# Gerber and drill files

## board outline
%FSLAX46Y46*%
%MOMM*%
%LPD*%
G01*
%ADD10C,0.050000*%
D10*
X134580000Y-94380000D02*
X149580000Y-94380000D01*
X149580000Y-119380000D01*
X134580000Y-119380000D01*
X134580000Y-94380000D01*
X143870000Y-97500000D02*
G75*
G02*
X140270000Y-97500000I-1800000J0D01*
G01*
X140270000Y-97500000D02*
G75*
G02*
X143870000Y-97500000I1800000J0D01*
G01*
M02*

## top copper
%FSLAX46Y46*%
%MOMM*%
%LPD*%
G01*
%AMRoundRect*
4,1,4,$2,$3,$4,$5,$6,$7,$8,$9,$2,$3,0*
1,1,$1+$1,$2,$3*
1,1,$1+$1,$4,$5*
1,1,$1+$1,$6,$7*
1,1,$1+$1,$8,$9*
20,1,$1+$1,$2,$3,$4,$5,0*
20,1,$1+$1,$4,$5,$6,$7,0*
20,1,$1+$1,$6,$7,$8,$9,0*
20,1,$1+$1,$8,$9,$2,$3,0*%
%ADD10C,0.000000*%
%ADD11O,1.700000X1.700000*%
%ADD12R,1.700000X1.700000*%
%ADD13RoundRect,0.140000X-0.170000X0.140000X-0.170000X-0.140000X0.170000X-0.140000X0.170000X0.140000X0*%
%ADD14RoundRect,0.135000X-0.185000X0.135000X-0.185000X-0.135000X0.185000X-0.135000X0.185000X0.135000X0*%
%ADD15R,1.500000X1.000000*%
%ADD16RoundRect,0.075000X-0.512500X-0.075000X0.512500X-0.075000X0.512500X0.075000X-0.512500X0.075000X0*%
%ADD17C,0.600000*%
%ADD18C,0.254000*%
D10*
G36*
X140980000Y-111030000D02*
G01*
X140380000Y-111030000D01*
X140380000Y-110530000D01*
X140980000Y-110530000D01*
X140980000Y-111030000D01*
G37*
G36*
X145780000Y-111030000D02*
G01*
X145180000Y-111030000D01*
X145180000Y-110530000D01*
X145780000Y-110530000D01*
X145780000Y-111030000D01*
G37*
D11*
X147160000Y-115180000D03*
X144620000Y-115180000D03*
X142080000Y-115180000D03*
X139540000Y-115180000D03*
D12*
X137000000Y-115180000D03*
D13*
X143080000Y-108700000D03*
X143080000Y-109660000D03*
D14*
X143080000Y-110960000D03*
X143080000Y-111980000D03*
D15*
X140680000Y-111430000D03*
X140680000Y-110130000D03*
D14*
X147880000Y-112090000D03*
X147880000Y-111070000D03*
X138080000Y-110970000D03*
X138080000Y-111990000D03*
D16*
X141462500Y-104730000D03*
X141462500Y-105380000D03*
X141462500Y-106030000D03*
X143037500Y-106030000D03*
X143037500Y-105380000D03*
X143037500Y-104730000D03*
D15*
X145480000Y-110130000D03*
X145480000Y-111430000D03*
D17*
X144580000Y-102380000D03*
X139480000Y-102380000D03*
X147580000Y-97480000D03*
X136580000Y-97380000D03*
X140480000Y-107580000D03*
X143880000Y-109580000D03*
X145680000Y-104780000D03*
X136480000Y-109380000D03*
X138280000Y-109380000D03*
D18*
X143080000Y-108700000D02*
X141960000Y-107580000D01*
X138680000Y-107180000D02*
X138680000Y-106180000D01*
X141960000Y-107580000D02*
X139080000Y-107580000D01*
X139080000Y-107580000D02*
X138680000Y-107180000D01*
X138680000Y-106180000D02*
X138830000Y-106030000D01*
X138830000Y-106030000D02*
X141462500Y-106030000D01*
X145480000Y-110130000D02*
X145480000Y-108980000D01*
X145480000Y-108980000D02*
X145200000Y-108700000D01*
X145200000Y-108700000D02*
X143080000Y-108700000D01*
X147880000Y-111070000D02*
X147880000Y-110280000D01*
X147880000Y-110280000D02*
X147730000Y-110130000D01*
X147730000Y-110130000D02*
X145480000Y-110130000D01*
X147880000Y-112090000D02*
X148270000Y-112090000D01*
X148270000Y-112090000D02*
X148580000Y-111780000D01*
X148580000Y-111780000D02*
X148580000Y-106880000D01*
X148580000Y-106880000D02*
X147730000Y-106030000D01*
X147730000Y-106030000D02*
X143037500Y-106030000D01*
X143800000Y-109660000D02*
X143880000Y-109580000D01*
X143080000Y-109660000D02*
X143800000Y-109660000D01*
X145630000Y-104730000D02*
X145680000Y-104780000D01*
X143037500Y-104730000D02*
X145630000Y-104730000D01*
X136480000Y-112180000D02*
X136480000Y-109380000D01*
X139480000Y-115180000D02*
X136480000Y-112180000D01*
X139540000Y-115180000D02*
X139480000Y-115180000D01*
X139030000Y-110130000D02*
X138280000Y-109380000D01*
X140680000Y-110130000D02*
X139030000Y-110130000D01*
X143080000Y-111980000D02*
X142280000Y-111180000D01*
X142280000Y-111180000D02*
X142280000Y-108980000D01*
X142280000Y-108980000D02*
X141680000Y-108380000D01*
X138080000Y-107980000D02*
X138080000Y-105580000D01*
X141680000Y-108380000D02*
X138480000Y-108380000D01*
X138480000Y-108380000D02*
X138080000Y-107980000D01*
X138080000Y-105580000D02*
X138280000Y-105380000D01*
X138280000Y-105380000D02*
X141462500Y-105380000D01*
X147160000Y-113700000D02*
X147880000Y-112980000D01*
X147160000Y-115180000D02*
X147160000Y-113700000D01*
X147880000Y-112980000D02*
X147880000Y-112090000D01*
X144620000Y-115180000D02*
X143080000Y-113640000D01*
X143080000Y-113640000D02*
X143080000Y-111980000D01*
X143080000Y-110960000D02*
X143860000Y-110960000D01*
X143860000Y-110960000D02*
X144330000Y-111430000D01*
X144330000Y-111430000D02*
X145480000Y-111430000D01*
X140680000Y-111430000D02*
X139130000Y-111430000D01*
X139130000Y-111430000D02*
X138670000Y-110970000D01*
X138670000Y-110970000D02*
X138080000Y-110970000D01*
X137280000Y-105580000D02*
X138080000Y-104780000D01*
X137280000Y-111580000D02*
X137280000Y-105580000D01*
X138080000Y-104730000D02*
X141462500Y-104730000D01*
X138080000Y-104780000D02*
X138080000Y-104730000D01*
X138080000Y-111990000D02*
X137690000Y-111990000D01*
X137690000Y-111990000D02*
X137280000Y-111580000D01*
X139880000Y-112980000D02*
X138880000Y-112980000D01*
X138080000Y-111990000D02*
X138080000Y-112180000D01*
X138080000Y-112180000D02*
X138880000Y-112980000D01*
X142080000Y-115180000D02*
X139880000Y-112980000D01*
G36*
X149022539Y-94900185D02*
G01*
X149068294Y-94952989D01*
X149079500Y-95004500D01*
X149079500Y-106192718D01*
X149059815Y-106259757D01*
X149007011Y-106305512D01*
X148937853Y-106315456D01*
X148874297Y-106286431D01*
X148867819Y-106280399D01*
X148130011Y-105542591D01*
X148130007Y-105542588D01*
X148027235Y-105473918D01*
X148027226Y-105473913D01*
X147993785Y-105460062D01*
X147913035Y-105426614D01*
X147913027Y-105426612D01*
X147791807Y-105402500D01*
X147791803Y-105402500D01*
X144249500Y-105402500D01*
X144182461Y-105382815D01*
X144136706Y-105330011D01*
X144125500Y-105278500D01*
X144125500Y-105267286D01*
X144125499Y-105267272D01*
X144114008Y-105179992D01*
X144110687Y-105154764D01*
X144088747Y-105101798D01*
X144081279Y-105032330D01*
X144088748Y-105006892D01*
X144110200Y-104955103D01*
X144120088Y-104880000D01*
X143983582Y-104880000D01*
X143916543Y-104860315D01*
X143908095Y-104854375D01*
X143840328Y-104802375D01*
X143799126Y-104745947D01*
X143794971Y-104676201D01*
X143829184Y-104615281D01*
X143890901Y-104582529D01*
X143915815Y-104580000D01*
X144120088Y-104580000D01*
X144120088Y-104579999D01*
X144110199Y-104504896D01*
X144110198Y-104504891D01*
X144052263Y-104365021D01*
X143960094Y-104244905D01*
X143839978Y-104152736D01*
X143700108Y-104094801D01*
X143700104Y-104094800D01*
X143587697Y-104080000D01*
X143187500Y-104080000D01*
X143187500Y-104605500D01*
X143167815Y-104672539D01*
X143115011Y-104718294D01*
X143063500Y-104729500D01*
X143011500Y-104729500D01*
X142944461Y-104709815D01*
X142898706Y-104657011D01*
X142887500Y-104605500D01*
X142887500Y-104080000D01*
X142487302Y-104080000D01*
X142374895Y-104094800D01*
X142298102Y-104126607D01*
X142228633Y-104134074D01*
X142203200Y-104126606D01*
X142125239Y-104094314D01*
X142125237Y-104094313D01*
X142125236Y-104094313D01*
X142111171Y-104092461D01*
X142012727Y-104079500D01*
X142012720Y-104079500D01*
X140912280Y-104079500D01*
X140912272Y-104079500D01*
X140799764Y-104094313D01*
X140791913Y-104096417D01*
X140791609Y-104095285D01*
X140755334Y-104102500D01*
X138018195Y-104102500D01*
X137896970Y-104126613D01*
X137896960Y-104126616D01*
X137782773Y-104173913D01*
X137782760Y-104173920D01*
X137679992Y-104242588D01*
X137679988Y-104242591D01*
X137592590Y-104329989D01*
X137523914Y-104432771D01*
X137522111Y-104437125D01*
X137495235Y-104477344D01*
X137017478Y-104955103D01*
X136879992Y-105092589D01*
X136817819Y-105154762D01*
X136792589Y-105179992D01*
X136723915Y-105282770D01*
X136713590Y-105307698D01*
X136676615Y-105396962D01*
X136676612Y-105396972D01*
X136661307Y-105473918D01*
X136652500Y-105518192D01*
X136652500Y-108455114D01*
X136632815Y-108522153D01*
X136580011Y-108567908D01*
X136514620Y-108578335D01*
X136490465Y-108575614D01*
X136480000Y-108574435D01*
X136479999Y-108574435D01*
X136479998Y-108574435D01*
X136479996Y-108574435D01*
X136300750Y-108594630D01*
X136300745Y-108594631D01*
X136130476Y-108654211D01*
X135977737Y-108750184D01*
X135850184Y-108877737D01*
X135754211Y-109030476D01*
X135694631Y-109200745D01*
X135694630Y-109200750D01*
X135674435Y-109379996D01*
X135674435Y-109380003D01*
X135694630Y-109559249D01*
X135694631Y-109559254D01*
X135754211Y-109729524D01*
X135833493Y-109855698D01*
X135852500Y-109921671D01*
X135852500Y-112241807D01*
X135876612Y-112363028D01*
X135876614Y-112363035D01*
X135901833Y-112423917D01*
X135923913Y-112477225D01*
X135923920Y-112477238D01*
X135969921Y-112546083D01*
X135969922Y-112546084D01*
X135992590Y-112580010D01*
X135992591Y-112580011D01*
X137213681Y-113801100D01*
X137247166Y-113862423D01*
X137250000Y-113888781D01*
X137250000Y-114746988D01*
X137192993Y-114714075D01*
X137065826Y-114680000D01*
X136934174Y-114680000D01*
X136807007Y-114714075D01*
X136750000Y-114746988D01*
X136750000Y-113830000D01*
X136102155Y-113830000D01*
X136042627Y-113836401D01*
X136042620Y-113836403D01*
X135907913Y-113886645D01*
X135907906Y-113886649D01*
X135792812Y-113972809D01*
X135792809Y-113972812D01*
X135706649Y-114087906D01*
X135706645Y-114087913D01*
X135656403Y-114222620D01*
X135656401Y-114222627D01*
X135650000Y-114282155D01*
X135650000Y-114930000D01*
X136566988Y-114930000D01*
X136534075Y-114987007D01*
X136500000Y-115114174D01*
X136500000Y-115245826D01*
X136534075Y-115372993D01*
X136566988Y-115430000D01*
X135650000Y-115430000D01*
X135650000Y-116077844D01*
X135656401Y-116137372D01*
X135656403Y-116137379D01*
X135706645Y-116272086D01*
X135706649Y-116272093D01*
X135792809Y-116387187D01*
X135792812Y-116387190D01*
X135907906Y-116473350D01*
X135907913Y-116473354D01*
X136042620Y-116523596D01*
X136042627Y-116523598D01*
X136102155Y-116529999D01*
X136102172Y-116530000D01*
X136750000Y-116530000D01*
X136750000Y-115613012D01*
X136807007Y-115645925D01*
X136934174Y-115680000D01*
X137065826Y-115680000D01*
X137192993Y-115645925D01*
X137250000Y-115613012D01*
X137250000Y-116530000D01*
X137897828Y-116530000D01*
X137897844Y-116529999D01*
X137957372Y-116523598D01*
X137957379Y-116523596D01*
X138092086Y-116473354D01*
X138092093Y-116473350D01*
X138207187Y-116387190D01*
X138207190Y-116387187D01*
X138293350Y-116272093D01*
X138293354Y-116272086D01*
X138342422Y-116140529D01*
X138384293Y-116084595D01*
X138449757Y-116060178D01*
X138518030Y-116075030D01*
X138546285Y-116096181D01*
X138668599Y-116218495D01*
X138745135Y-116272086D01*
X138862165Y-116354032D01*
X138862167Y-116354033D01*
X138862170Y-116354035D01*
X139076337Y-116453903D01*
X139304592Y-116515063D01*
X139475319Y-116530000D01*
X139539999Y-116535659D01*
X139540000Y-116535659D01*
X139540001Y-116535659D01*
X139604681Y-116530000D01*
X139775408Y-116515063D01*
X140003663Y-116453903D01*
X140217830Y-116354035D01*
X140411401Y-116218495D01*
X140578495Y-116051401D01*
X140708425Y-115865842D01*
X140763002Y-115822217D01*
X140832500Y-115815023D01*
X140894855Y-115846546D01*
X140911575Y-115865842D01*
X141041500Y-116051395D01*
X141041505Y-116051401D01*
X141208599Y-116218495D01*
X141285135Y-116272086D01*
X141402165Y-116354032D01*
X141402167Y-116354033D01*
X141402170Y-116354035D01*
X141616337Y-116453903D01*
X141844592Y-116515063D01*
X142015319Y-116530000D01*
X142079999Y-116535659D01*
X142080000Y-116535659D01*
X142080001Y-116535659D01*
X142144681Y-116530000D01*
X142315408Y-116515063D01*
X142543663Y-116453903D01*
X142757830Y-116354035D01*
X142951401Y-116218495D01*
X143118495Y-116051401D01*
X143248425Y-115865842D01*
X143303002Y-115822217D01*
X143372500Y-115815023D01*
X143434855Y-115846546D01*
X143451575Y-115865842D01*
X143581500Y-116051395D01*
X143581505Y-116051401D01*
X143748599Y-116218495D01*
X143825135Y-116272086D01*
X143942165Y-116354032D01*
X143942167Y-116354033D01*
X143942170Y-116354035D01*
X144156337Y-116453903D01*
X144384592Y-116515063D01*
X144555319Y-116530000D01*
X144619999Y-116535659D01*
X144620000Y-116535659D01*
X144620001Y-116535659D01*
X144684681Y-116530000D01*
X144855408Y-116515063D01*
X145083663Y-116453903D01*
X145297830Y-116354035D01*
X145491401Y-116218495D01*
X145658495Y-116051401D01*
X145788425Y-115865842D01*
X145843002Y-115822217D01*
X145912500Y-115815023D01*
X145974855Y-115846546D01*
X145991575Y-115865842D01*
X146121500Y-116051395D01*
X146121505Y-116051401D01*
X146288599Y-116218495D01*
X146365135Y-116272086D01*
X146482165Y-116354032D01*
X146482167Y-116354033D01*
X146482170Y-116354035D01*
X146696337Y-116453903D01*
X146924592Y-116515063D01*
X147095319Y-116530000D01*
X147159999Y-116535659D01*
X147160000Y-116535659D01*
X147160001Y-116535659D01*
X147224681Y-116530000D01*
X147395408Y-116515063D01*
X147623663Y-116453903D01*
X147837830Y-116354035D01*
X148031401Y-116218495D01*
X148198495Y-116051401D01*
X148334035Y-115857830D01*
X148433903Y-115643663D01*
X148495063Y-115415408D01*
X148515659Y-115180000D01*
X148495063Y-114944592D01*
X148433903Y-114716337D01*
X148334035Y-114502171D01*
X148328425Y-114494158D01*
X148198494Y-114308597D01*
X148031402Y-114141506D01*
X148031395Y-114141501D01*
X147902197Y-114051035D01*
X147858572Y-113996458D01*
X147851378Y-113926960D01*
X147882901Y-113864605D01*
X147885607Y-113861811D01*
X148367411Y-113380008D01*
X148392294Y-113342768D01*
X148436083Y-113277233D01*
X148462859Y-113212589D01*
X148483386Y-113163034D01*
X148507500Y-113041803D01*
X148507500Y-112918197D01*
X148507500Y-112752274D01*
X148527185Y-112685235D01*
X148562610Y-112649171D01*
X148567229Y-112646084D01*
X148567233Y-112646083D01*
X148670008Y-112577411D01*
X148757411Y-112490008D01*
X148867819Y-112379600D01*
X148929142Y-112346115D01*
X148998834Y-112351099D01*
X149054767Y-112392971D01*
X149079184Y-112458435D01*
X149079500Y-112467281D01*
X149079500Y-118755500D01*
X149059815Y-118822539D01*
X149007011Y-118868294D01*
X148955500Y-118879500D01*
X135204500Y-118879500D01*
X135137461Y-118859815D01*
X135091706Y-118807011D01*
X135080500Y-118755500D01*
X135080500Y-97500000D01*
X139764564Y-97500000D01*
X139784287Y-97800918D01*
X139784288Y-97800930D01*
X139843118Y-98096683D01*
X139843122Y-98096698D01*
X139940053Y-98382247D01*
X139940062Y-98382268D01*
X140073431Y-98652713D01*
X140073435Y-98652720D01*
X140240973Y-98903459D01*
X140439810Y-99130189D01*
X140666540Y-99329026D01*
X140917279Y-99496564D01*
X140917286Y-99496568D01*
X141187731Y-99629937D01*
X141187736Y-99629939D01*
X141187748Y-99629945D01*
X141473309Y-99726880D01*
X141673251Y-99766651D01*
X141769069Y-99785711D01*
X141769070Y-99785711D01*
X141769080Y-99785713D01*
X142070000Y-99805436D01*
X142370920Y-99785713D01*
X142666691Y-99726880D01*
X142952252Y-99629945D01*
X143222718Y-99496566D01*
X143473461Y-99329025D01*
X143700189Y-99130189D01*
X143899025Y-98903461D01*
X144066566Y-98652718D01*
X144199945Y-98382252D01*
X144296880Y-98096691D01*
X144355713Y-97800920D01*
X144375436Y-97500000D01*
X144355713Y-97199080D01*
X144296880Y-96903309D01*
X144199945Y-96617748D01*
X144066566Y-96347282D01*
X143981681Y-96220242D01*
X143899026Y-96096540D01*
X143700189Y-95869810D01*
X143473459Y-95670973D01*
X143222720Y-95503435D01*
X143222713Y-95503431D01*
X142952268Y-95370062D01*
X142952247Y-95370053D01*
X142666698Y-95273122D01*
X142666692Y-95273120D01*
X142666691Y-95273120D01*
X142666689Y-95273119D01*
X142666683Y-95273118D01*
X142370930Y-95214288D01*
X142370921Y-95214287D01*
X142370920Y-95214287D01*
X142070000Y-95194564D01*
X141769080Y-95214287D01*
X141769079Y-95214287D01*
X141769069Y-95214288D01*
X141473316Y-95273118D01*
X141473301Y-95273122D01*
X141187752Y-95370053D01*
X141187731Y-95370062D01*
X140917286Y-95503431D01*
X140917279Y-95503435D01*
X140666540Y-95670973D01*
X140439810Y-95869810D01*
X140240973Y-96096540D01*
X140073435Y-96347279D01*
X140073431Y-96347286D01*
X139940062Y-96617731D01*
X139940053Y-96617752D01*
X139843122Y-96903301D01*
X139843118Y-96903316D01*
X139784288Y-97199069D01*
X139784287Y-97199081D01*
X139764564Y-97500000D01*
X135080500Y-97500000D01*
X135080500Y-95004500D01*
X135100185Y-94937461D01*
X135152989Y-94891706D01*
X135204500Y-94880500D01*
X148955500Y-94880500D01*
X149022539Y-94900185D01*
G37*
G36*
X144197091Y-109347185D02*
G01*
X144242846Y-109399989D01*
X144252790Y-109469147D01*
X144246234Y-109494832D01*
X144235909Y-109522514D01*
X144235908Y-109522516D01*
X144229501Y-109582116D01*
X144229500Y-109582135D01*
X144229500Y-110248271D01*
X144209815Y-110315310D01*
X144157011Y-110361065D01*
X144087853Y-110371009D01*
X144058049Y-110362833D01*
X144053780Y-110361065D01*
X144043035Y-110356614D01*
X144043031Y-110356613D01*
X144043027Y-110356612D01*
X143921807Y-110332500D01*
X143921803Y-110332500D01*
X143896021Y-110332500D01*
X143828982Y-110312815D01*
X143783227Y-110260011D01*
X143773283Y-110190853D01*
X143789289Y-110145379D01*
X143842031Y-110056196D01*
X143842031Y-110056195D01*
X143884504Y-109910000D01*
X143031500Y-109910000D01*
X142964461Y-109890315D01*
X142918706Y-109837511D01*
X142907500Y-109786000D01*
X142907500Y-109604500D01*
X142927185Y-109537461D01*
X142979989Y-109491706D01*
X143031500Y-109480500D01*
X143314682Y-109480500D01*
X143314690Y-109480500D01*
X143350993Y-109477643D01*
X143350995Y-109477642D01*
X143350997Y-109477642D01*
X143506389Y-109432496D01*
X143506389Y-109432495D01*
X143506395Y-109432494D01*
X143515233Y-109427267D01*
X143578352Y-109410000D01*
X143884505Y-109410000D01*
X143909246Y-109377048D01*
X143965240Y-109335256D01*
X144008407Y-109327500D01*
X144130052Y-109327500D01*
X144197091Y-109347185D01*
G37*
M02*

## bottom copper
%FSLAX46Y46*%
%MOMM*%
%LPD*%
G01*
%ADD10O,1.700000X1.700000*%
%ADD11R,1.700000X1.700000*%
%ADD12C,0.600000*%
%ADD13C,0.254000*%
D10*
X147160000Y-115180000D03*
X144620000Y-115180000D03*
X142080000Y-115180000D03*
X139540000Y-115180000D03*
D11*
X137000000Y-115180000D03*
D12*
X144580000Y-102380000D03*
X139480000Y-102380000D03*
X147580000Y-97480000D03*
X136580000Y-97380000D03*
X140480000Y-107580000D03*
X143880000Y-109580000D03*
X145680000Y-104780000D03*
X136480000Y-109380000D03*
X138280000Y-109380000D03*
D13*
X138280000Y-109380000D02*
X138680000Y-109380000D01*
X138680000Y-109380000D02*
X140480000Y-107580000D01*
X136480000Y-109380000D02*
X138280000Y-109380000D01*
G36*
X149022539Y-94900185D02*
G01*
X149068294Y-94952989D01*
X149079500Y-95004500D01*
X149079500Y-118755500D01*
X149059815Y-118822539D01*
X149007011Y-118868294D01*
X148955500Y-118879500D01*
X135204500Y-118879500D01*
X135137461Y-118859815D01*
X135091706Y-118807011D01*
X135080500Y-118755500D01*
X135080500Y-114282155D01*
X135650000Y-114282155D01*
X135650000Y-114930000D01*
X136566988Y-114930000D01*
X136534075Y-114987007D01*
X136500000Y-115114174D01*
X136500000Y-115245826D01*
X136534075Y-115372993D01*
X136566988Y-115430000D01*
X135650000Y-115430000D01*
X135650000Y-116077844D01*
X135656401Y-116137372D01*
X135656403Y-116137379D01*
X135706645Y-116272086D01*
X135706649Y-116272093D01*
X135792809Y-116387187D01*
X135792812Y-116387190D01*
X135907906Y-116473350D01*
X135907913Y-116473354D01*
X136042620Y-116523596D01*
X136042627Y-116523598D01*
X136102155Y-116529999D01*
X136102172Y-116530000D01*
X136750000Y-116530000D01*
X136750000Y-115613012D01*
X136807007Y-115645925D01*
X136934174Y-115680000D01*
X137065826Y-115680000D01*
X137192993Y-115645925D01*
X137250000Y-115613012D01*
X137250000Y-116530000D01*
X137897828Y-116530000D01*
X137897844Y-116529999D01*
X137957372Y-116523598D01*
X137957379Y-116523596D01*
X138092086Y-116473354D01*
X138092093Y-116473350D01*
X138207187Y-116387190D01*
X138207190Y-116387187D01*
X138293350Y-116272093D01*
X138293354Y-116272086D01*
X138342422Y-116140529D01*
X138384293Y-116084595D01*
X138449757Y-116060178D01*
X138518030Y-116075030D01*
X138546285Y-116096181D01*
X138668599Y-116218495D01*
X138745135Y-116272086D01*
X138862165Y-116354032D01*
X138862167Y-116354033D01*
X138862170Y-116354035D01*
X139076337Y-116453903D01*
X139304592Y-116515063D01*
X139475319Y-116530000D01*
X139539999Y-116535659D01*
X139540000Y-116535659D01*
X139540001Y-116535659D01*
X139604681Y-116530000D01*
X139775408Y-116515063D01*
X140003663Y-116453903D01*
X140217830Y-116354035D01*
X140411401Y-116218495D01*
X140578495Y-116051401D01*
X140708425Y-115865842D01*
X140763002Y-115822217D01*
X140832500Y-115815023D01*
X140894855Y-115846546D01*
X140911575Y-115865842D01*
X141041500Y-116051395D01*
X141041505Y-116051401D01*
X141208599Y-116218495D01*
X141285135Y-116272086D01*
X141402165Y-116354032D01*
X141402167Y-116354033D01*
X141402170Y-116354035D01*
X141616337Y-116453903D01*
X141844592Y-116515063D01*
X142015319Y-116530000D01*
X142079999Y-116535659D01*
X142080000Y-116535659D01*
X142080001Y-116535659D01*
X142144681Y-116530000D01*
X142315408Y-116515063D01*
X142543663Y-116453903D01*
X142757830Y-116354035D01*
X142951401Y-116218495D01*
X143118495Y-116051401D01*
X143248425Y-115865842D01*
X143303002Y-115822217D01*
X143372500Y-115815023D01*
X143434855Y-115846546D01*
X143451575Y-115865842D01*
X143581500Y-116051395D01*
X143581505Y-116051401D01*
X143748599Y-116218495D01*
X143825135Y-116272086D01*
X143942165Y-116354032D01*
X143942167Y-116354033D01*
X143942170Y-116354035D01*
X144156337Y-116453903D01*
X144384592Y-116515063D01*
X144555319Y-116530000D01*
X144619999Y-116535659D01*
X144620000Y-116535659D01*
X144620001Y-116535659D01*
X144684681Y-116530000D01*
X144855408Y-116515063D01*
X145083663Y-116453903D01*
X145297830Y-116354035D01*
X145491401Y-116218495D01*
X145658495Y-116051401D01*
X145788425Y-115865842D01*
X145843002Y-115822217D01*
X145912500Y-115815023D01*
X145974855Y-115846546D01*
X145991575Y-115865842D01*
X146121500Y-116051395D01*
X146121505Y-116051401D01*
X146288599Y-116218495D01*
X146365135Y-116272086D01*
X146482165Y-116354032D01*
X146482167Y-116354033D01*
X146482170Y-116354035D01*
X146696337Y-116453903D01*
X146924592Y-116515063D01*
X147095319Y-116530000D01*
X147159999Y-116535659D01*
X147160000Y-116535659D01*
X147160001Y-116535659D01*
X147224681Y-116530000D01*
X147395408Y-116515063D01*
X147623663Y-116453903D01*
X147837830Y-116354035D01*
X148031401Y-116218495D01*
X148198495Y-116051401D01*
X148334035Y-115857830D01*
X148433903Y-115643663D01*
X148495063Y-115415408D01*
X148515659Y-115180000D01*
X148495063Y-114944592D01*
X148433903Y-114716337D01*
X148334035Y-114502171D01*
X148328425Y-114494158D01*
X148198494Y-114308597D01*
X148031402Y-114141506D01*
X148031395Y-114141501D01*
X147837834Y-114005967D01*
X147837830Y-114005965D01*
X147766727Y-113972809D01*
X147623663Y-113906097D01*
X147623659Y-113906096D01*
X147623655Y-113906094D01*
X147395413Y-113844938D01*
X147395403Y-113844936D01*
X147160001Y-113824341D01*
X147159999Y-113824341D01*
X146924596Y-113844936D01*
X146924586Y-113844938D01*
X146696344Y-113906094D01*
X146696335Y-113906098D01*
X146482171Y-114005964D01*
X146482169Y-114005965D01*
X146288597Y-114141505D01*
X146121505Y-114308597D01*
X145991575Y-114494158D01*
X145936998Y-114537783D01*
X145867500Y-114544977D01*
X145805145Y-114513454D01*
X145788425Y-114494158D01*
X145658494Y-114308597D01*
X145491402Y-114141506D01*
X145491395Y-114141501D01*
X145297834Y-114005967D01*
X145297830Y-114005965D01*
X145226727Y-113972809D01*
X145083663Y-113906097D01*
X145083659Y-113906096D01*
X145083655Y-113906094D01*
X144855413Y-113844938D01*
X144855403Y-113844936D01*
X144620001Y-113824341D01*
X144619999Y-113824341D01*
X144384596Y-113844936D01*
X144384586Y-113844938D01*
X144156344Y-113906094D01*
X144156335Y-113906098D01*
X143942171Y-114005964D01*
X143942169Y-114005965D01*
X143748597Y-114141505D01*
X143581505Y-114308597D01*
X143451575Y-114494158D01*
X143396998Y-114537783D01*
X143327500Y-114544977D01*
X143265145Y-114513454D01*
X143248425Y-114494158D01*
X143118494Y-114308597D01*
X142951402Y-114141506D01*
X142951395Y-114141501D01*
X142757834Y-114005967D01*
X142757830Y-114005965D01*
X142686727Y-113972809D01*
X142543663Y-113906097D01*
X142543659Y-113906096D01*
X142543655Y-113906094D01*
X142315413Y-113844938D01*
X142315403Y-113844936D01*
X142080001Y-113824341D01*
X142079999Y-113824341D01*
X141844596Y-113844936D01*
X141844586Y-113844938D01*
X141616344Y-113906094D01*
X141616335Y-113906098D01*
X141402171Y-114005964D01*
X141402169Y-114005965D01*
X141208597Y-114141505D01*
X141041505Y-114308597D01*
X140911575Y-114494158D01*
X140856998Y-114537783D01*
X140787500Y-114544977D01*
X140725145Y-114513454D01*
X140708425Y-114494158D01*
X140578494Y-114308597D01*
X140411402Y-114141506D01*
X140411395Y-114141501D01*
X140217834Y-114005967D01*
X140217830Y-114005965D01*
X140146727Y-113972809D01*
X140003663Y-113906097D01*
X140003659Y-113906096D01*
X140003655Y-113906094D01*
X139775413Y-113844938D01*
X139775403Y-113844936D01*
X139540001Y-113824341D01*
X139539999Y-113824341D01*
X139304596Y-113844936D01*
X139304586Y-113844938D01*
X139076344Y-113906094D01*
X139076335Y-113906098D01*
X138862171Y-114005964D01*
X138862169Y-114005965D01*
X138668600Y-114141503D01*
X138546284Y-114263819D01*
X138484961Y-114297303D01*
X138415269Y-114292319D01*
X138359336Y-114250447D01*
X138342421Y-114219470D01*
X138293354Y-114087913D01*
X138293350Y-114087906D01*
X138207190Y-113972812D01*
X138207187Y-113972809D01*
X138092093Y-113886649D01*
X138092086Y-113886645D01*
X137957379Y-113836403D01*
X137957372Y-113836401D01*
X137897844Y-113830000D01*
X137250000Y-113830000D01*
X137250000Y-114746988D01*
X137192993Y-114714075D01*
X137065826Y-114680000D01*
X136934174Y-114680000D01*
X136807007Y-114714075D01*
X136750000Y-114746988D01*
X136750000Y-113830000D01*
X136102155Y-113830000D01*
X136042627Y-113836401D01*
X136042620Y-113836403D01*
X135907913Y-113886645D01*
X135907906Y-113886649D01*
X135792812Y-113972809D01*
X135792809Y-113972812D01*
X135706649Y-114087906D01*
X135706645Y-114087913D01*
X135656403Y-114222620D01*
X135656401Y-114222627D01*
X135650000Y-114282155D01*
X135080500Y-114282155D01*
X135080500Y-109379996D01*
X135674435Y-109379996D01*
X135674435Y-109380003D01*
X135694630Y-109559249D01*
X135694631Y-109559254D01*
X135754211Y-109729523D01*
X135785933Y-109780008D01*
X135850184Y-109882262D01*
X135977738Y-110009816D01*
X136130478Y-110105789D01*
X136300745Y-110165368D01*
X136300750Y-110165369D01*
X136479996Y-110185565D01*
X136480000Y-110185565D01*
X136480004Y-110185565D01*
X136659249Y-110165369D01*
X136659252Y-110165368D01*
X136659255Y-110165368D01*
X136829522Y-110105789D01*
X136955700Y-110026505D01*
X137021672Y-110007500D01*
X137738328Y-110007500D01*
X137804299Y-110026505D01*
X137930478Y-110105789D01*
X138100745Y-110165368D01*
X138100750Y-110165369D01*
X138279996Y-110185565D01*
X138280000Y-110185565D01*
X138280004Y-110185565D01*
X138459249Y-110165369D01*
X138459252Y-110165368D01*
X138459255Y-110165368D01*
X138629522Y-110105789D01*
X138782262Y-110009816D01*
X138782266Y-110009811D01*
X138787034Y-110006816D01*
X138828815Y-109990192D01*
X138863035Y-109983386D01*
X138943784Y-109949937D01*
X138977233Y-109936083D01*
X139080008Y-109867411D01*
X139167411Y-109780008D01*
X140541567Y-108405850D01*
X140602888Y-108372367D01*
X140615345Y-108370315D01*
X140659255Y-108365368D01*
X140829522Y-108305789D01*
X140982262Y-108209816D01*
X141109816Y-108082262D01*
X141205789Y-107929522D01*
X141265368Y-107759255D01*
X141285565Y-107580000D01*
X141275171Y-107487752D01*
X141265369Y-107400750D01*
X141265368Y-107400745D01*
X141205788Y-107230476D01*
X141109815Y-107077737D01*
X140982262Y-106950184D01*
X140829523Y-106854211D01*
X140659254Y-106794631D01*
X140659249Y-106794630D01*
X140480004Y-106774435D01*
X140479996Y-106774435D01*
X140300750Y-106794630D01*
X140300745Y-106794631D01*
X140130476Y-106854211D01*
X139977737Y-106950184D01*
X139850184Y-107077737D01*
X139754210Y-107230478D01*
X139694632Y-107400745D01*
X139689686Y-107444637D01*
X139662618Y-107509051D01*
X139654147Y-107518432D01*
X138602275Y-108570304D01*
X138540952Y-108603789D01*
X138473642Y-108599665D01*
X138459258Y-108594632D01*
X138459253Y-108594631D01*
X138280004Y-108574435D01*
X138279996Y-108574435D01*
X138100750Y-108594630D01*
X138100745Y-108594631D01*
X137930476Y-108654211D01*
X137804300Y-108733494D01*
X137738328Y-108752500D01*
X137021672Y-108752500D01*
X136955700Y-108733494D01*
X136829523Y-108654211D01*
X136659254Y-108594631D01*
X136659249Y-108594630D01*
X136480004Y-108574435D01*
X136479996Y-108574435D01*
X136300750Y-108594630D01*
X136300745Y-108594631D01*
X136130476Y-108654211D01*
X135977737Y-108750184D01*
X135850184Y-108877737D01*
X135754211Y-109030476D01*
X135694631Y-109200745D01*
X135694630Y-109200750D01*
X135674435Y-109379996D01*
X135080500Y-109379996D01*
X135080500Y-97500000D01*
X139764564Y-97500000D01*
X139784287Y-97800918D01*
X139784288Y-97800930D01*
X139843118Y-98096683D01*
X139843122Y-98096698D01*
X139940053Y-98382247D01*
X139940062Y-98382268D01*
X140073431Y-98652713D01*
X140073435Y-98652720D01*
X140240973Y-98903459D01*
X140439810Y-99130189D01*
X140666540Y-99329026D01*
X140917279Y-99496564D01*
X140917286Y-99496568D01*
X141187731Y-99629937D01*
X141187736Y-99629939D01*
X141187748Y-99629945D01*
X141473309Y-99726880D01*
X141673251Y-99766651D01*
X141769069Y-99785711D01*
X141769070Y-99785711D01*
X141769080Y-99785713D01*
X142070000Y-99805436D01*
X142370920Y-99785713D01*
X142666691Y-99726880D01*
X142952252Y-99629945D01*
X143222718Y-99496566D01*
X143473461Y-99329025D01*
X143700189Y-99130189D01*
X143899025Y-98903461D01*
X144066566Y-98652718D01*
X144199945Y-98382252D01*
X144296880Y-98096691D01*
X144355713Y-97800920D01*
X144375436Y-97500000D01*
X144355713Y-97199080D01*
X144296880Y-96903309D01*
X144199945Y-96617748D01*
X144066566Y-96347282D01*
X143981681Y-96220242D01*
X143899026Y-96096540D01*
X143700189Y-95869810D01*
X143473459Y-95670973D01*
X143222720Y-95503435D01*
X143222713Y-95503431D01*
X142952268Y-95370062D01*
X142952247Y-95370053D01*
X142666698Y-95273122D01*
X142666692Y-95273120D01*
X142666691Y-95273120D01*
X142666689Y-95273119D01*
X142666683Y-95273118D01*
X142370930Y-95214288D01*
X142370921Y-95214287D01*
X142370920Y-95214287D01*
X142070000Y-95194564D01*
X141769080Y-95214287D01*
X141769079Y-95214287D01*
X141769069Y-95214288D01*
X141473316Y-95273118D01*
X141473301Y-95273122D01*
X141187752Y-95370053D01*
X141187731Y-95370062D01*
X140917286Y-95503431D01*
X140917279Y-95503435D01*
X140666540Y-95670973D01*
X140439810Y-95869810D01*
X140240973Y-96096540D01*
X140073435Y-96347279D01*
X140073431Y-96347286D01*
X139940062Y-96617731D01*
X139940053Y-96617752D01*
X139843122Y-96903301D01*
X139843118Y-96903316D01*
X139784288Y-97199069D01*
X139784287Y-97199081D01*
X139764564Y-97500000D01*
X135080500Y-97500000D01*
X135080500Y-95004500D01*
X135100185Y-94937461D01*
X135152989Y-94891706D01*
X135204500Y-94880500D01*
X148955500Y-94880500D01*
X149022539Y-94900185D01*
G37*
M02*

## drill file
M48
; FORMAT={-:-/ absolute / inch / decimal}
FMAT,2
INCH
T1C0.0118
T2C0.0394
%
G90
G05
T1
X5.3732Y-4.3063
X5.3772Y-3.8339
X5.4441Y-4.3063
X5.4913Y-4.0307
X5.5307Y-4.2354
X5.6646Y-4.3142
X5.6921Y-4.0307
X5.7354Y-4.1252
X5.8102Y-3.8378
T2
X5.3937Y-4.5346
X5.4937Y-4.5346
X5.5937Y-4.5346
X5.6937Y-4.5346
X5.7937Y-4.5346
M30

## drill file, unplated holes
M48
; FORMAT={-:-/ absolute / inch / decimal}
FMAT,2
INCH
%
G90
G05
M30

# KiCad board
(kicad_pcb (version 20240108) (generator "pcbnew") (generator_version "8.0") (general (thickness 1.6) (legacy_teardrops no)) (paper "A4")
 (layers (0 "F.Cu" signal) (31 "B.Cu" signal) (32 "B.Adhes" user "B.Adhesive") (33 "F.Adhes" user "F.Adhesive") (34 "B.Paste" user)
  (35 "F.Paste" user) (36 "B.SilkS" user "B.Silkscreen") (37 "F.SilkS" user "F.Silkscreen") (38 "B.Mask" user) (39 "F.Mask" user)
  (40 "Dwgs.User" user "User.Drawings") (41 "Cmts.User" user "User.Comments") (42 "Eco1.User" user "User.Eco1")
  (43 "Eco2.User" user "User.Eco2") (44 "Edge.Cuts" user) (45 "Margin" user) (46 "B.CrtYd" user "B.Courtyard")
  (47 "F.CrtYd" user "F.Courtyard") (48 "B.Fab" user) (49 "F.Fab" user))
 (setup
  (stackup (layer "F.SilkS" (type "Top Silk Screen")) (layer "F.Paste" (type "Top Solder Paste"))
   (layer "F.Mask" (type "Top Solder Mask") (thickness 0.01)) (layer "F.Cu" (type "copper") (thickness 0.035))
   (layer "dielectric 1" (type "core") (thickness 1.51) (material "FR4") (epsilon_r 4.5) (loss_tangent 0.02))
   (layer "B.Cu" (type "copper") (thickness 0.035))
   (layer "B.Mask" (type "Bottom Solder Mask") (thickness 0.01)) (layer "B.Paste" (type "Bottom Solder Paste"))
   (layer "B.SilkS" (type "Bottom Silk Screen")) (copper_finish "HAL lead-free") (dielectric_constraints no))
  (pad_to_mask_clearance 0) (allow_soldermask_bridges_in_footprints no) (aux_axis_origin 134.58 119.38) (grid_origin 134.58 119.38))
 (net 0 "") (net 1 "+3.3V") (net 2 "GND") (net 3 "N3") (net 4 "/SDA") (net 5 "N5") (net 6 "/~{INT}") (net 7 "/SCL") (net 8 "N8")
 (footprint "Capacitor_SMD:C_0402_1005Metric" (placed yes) (layer "F.Cu") (at 143.08 109.18 -90)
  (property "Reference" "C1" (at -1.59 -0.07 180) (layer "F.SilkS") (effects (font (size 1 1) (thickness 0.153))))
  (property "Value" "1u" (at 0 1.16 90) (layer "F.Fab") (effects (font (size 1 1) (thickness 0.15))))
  (pad "1" smd roundrect (at -0.48 0 270) (size 0.56 0.62) (layers "F.Cu" "F.Paste" "F.Mask") (roundrect_rratio 0.25) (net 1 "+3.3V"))
  (pad "2" smd roundrect (at 0.48 0 270) (size 0.56 0.62) (layers "F.Cu" "F.Paste" "F.Mask") (roundrect_rratio 0.25) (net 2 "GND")))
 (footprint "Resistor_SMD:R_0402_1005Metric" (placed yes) (layer "F.Cu") (at 143.08 111.47 -90)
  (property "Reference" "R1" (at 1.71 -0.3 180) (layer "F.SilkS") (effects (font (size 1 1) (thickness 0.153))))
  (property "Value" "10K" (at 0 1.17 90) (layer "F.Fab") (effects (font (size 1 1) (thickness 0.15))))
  (pad "1" smd roundrect (at -0.51 0 270) (size 0.54 0.64) (layers "F.Cu" "F.Paste" "F.Mask") (roundrect_rratio 0.25) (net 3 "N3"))
  (pad "2" smd roundrect (at 0.51 0 270) (size 0.54 0.64) (layers "F.Cu" "F.Paste" "F.Mask") (roundrect_rratio 0.25) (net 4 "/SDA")))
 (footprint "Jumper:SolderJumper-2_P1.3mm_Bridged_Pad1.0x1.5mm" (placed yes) (layer "F.Cu") (at 140.68 110.78 90)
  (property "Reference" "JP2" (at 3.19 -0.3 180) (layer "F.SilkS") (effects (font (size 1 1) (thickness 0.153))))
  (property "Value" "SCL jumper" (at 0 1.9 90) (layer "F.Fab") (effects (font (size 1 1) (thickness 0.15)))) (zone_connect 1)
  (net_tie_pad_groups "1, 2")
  (fp_poly (pts (xy -0.25 -0.3) (xy 0.25 -0.3) (xy 0.25 0.3) (xy -0.25 0.3)) (stroke (width 0) (type solid)) (fill solid) (layer "F.Cu"))
  (pad "1" smd rect (at -0.65 0 90) (size 1 1.5) (layers "F.Cu" "F.Mask") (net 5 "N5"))
  (pad "2" smd rect (at 0.65 0 90) (size 1 1.5) (layers "F.Cu" "F.Mask") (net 1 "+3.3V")))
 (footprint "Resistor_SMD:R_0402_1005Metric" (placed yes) (layer "F.Cu") (at 147.88 111.58 -90)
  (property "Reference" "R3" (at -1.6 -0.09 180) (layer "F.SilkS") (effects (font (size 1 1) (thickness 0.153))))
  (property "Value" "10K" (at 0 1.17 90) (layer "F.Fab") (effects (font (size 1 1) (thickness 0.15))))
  (pad "1" smd roundrect (at -0.51 0 270) (size 0.54 0.64) (layers "F.Cu" "F.Paste" "F.Mask") (roundrect_rratio 0.25) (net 1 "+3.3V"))
  (pad "2" smd roundrect (at 0.51 0 270) (size 0.54 0.64) (layers "F.Cu" "F.Paste" "F.Mask") (roundrect_rratio 0.25) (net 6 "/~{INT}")))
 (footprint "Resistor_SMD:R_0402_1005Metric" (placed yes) (layer "F.Cu") (at 138.08 111.48 -90)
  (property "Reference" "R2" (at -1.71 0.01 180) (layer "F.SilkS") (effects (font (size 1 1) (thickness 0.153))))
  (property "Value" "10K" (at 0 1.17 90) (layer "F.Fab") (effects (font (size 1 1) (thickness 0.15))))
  (pad "1" smd roundrect (at -0.51 0 270) (size 0.54 0.64) (layers "F.Cu" "F.Paste" "F.Mask") (roundrect_rratio 0.25) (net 5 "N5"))
  (pad "2" smd roundrect (at 0.51 0 270) (size 0.54 0.64) (layers "F.Cu" "F.Paste" "F.Mask") (roundrect_rratio 0.25) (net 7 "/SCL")))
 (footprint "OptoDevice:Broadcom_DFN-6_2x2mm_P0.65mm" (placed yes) (layer "F.Cu") (at 142.25 105.38)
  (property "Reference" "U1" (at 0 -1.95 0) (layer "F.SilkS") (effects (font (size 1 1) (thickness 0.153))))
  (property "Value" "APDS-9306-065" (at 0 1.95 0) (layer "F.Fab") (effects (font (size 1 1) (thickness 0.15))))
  (pad "1" smd roundrect (at -0.7875 -0.65) (size 1.175 0.3) (layers "F.Cu" "F.Paste" "F.Mask") (roundrect_rratio 0.25) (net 7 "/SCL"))
  (pad "2" smd roundrect (at -0.7875 0) (size 1.175 0.3) (layers "F.Cu" "F.Paste" "F.Mask") (roundrect_rratio 0.25) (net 4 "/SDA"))
  (pad "3" smd roundrect (at -0.7875 0.65) (size 1.175 0.3) (layers "F.Cu" "F.Paste" "F.Mask") (roundrect_rratio 0.25) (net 1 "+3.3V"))
  (pad "4" smd roundrect (at 0.7875 0.65) (size 1.175 0.3) (layers "F.Cu" "F.Paste" "F.Mask") (roundrect_rratio 0.25) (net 6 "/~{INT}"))
  (pad "5" smd roundrect (at 0.7875 0) (size 1.175 0.3) (layers "F.Cu" "F.Paste" "F.Mask") (roundrect_rratio 0.25) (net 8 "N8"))
  (pad "6" smd roundrect (at 0.7875 -0.65) (size 1.175 0.3) (layers "F.Cu" "F.Paste" "F.Mask") (roundrect_rratio 0.25) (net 2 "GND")))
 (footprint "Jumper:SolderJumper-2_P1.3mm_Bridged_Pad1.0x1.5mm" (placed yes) (layer "F.Cu") (at 145.48 110.78 90)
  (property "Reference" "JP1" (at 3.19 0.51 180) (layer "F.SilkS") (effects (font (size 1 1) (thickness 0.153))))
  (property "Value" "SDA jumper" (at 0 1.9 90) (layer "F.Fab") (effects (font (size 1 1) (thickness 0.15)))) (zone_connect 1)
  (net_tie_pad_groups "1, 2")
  (fp_poly (pts (xy -0.25 -0.3) (xy 0.25 -0.3) (xy 0.25 0.3) (xy -0.25 0.3)) (stroke (width 0) (type solid)) (fill solid) (layer "F.Cu"))
  (pad "1" smd rect (at -0.65 0 90) (size 1 1.5) (layers "F.Cu" "F.Mask") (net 3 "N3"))
  (pad "2" smd rect (at 0.65 0 90) (size 1 1.5) (layers "F.Cu" "F.Mask") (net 1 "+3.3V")))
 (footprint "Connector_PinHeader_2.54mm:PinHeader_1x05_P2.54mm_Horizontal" (layer "B.Cu") (at 137 115.18 -90)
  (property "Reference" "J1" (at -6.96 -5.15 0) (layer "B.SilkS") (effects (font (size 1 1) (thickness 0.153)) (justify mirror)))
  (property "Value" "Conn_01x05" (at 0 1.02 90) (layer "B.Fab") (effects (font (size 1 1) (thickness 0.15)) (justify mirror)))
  (pad "1" thru_hole rect (at 0 0 270) (size 1.7 1.7) (drill 1) (layers "*.Cu" "*.Mask") (remove_unused_layers no) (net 2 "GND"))
  (pad "2" thru_hole oval (at 0 -2.54 270) (size 1.7 1.7) (drill 1) (layers "*.Cu" "*.Mask") (remove_unused_layers no) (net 1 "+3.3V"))
  (pad "3" thru_hole oval (at 0 -5.08 270) (size 1.7 1.7) (drill 1) (layers "*.Cu" "*.Mask") (remove_unused_layers no) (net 7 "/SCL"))
  (pad "4" thru_hole oval (at 0 -7.62 270) (size 1.7 1.7) (drill 1) (layers "*.Cu" "*.Mask") (remove_unused_layers no) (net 4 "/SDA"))
  (pad "5" thru_hole oval (at 0 -10.16 270) (size 1.7 1.7) (drill 1) (layers "*.Cu" "*.Mask") (remove_unused_layers no) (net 6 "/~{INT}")))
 (gr_rect (start 134.58 94.38) (end 149.58 119.38) (stroke (width 0.05) (type default)) (fill none) (layer "Edge.Cuts"))
 (gr_circle (center 142.07 97.5) (end 143.87 97.5) (stroke (width 0.05) (type default)) (fill none) (layer "Edge.Cuts"))
 (segment (start 147.88 111.07) (end 147.88 110.28) (width 0.254) (layer "F.Cu") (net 1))
 (segment (start 143.08 108.7) (end 141.96 107.58) (width 0.254) (layer "F.Cu") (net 1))
 (segment (start 136.48 112.18) (end 136.48 109.38) (width 0.254) (layer "F.Cu") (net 1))
 (segment (start 139.03 110.13) (end 138.28 109.38) (width 0.254) (layer "F.Cu") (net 1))
 (segment (start 138.68 106.18) (end 138.83 106.03) (width 0.254) (layer "F.Cu") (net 1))
 (segment (start 140.68 110.13) (end 139.03 110.13) (width 0.254) (layer "F.Cu") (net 1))
 (segment (start 139.54 115.18) (end 139.48 115.18) (width 0.254) (layer "F.Cu") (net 1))
 (segment (start 139.48 115.18) (end 136.48 112.18) (width 0.254) (layer "F.Cu") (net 1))
 (segment (start 145.48 108.98) (end 145.2 108.7) (width 0.254) (layer "F.Cu") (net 1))
 (segment (start 141.96 107.58) (end 139.08 107.58) (width 0.254) (layer "F.Cu") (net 1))
 (segment (start 138.83 106.03) (end 141.4625 106.03) (width 0.254) (layer "F.Cu") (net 1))
 (segment (start 145.2 108.7) (end 143.08 108.7) (width 0.254) (layer "F.Cu") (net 1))
 (segment (start 138.68 107.18) (end 138.68 106.18) (width 0.254) (layer "F.Cu") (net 1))
 (segment (start 147.73 110.13) (end 145.48 110.13) (width 0.254) (layer "F.Cu") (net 1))
 (segment (start 139.08 107.58) (end 138.68 107.18) (width 0.254) (layer "F.Cu") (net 1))
 (segment (start 145.48 110.13) (end 145.48 108.98) (width 0.254) (layer "F.Cu") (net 1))
 (segment (start 147.88 110.28) (end 147.73 110.13) (width 0.254) (layer "F.Cu") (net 1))
 (via (at 138.28 109.38) (size 0.6) (drill 0.3) (layers "F.Cu" "B.Cu") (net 1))
 (via (at 136.48 109.38) (size 0.6) (drill 0.3) (layers "F.Cu" "B.Cu") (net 1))
 (via (at 140.48 107.58) (size 0.6) (drill 0.3) (layers "F.Cu" "B.Cu") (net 1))
 (segment (start 136.48 109.38) (end 138.28 109.38) (width 0.254) (layer "B.Cu") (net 1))
 (segment (start 138.28 109.38) (end 138.68 109.38) (width 0.254) (layer "B.Cu") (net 1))
 (segment (start 138.68 109.38) (end 140.48 107.58) (width 0.254) (layer "B.Cu") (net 1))
 (segment (start 143.8 109.66) (end 143.88 109.58) (width 0.254) (layer "F.Cu") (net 2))
 (segment (start 145.63 104.73) (end 145.68 104.78) (width 0.254) (layer "F.Cu") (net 2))
 (segment (start 143.0375 104.73) (end 145.63 104.73) (width 0.254) (layer "F.Cu") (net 2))
 (segment (start 143.08 109.66) (end 143.8 109.66) (width 0.254) (layer "F.Cu") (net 2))
 (via (at 145.68 104.78) (size 0.6) (drill 0.3) (layers "F.Cu" "B.Cu") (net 2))
 (via (at 147.58 97.48) (size 0.6) (drill 0.3) (layers "F.Cu" "B.Cu") (free yes) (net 2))
 (via (at 139.48 102.38) (size 0.6) (drill 0.3) (layers "F.Cu" "B.Cu") (free yes) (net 2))
 (via (at 144.58 102.38) (size 0.6) (drill 0.3) (layers "F.Cu" "B.Cu") (free yes) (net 2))
 (via (at 143.88 109.58) (size 0.6) (drill 0.3) (layers "F.Cu" "B.Cu") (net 2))
 (via (at 136.58 97.38) (size 0.6) (drill 0.3) (layers "F.Cu" "B.Cu") (free yes) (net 2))
 (segment (start 147.88 112.98) (end 147.88 112.09) (width 0.254) (layer "F.Cu") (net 6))
 (segment (start 148.58 111.78) (end 148.58 106.88) (width 0.254) (layer "F.Cu") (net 6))
 (segment (start 148.58 106.88) (end 147.73 106.03) (width 0.254) (layer "F.Cu") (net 6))
 (segment (start 148.27 112.09) (end 148.58 111.78) (width 0.254) (layer "F.Cu") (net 6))
 (segment (start 147.16 115.18) (end 147.16 113.7) (width 0.254) (layer "F.Cu") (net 6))
 (segment (start 147.16 113.7) (end 147.88 112.98) (width 0.254) (layer "F.Cu") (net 6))
 (segment (start 147.73 106.03) (end 143.0375 106.03) (width 0.254) (layer "F.Cu") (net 6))
 (segment (start 147.88 112.09) (end 148.27 112.09) (width 0.254) (layer "F.Cu") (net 6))
 (segment (start 138.08 111.99) (end 138.08 112.18) (width 0.254) (layer "F.Cu") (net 7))
 (segment (start 139.88 112.98) (end 138.88 112.98) (width 0.254) (layer "F.Cu") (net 7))
 (segment (start 137.28 111.58) (end 137.28 105.58) (width 0.254) (layer "F.Cu") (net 7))
 (segment (start 137.28 105.58) (end 138.08 104.78) (width 0.254) (layer "F.Cu") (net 7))
 (segment (start 138.08 111.99) (end 137.69 111.99) (width 0.254) (layer "F.Cu") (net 7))
 (segment (start 142.08 115.18) (end 139.88 112.98) (width 0.254) (layer "F.Cu") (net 7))
 (segment (start 137.69 111.99) (end 137.28 111.58) (width 0.254) (layer "F.Cu") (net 7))
 (segment (start 138.08 104.78) (end 138.08 104.73) (width 0.254) (layer "F.Cu") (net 7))
 (segment (start 138.08 112.18) (end 138.88 112.98) (width 0.254) (layer "F.Cu") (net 7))
 (segment (start 138.08 104.73) (end 141.4625 104.73) (width 0.254) (layer "F.Cu") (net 7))
 (segment (start 143.08 111.98) (end 142.28 111.18) (width 0.254) (layer "F.Cu") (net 4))
 (segment (start 138.28 105.38) (end 141.4625 105.38) (width 0.254) (layer "F.Cu") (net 4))
 (segment (start 141.68 108.38) (end 138.48 108.38) (width 0.254) (layer "F.Cu") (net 4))
 (segment (start 142.28 111.18) (end 142.28 108.98) (width 0.254) (layer "F.Cu") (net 4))
 (segment (start 138.48 108.38) (end 138.08 107.98) (width 0.254) (layer "F.Cu") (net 4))
 (segment (start 142.28 108.98) (end 141.68 108.38) (width 0.254) (layer "F.Cu") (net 4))
 (segment (start 138.08 107.98) (end 138.08 105.58) (width 0.254) (layer "F.Cu") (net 4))
 (segment (start 138.08 105.58) (end 138.28 105.38) (width 0.254) (layer "F.Cu") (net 4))
 (segment (start 144.62 115.18) (end 143.08 113.64) (width 0.254) (layer "F.Cu") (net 4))
 (segment (start 143.08 113.64) (end 143.08 111.98) (width 0.254) (layer "F.Cu") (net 4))
 (segment (start 143.86 110.96) (end 144.33 111.43) (width 0.254) (layer "F.Cu") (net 3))
 (segment (start 144.33 111.43) (end 145.48 111.43) (width 0.254) (layer "F.Cu") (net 3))
 (segment (start 143.08 110.96) (end 143.86 110.96) (width 0.254) (layer "F.Cu") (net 3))
 (segment (start 140.68 111.43) (end 139.13 111.43) (width 0.254) (layer "F.Cu") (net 5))
 (segment (start 138.67 110.97) (end 138.08 110.97) (width 0.254) (layer "F.Cu") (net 5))
 (segment (start 139.13 111.43) (end 138.67 110.97) (width 0.254) (layer "F.Cu") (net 5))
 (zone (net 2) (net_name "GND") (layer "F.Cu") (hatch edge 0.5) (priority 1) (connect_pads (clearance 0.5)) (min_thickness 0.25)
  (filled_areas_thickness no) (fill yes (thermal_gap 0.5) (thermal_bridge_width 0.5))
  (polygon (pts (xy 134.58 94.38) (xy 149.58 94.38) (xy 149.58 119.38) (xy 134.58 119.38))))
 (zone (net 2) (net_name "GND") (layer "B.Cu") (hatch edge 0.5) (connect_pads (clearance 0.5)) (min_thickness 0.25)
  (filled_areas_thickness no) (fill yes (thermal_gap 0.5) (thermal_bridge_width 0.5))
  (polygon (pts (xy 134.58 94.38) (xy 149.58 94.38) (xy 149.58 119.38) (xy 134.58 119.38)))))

